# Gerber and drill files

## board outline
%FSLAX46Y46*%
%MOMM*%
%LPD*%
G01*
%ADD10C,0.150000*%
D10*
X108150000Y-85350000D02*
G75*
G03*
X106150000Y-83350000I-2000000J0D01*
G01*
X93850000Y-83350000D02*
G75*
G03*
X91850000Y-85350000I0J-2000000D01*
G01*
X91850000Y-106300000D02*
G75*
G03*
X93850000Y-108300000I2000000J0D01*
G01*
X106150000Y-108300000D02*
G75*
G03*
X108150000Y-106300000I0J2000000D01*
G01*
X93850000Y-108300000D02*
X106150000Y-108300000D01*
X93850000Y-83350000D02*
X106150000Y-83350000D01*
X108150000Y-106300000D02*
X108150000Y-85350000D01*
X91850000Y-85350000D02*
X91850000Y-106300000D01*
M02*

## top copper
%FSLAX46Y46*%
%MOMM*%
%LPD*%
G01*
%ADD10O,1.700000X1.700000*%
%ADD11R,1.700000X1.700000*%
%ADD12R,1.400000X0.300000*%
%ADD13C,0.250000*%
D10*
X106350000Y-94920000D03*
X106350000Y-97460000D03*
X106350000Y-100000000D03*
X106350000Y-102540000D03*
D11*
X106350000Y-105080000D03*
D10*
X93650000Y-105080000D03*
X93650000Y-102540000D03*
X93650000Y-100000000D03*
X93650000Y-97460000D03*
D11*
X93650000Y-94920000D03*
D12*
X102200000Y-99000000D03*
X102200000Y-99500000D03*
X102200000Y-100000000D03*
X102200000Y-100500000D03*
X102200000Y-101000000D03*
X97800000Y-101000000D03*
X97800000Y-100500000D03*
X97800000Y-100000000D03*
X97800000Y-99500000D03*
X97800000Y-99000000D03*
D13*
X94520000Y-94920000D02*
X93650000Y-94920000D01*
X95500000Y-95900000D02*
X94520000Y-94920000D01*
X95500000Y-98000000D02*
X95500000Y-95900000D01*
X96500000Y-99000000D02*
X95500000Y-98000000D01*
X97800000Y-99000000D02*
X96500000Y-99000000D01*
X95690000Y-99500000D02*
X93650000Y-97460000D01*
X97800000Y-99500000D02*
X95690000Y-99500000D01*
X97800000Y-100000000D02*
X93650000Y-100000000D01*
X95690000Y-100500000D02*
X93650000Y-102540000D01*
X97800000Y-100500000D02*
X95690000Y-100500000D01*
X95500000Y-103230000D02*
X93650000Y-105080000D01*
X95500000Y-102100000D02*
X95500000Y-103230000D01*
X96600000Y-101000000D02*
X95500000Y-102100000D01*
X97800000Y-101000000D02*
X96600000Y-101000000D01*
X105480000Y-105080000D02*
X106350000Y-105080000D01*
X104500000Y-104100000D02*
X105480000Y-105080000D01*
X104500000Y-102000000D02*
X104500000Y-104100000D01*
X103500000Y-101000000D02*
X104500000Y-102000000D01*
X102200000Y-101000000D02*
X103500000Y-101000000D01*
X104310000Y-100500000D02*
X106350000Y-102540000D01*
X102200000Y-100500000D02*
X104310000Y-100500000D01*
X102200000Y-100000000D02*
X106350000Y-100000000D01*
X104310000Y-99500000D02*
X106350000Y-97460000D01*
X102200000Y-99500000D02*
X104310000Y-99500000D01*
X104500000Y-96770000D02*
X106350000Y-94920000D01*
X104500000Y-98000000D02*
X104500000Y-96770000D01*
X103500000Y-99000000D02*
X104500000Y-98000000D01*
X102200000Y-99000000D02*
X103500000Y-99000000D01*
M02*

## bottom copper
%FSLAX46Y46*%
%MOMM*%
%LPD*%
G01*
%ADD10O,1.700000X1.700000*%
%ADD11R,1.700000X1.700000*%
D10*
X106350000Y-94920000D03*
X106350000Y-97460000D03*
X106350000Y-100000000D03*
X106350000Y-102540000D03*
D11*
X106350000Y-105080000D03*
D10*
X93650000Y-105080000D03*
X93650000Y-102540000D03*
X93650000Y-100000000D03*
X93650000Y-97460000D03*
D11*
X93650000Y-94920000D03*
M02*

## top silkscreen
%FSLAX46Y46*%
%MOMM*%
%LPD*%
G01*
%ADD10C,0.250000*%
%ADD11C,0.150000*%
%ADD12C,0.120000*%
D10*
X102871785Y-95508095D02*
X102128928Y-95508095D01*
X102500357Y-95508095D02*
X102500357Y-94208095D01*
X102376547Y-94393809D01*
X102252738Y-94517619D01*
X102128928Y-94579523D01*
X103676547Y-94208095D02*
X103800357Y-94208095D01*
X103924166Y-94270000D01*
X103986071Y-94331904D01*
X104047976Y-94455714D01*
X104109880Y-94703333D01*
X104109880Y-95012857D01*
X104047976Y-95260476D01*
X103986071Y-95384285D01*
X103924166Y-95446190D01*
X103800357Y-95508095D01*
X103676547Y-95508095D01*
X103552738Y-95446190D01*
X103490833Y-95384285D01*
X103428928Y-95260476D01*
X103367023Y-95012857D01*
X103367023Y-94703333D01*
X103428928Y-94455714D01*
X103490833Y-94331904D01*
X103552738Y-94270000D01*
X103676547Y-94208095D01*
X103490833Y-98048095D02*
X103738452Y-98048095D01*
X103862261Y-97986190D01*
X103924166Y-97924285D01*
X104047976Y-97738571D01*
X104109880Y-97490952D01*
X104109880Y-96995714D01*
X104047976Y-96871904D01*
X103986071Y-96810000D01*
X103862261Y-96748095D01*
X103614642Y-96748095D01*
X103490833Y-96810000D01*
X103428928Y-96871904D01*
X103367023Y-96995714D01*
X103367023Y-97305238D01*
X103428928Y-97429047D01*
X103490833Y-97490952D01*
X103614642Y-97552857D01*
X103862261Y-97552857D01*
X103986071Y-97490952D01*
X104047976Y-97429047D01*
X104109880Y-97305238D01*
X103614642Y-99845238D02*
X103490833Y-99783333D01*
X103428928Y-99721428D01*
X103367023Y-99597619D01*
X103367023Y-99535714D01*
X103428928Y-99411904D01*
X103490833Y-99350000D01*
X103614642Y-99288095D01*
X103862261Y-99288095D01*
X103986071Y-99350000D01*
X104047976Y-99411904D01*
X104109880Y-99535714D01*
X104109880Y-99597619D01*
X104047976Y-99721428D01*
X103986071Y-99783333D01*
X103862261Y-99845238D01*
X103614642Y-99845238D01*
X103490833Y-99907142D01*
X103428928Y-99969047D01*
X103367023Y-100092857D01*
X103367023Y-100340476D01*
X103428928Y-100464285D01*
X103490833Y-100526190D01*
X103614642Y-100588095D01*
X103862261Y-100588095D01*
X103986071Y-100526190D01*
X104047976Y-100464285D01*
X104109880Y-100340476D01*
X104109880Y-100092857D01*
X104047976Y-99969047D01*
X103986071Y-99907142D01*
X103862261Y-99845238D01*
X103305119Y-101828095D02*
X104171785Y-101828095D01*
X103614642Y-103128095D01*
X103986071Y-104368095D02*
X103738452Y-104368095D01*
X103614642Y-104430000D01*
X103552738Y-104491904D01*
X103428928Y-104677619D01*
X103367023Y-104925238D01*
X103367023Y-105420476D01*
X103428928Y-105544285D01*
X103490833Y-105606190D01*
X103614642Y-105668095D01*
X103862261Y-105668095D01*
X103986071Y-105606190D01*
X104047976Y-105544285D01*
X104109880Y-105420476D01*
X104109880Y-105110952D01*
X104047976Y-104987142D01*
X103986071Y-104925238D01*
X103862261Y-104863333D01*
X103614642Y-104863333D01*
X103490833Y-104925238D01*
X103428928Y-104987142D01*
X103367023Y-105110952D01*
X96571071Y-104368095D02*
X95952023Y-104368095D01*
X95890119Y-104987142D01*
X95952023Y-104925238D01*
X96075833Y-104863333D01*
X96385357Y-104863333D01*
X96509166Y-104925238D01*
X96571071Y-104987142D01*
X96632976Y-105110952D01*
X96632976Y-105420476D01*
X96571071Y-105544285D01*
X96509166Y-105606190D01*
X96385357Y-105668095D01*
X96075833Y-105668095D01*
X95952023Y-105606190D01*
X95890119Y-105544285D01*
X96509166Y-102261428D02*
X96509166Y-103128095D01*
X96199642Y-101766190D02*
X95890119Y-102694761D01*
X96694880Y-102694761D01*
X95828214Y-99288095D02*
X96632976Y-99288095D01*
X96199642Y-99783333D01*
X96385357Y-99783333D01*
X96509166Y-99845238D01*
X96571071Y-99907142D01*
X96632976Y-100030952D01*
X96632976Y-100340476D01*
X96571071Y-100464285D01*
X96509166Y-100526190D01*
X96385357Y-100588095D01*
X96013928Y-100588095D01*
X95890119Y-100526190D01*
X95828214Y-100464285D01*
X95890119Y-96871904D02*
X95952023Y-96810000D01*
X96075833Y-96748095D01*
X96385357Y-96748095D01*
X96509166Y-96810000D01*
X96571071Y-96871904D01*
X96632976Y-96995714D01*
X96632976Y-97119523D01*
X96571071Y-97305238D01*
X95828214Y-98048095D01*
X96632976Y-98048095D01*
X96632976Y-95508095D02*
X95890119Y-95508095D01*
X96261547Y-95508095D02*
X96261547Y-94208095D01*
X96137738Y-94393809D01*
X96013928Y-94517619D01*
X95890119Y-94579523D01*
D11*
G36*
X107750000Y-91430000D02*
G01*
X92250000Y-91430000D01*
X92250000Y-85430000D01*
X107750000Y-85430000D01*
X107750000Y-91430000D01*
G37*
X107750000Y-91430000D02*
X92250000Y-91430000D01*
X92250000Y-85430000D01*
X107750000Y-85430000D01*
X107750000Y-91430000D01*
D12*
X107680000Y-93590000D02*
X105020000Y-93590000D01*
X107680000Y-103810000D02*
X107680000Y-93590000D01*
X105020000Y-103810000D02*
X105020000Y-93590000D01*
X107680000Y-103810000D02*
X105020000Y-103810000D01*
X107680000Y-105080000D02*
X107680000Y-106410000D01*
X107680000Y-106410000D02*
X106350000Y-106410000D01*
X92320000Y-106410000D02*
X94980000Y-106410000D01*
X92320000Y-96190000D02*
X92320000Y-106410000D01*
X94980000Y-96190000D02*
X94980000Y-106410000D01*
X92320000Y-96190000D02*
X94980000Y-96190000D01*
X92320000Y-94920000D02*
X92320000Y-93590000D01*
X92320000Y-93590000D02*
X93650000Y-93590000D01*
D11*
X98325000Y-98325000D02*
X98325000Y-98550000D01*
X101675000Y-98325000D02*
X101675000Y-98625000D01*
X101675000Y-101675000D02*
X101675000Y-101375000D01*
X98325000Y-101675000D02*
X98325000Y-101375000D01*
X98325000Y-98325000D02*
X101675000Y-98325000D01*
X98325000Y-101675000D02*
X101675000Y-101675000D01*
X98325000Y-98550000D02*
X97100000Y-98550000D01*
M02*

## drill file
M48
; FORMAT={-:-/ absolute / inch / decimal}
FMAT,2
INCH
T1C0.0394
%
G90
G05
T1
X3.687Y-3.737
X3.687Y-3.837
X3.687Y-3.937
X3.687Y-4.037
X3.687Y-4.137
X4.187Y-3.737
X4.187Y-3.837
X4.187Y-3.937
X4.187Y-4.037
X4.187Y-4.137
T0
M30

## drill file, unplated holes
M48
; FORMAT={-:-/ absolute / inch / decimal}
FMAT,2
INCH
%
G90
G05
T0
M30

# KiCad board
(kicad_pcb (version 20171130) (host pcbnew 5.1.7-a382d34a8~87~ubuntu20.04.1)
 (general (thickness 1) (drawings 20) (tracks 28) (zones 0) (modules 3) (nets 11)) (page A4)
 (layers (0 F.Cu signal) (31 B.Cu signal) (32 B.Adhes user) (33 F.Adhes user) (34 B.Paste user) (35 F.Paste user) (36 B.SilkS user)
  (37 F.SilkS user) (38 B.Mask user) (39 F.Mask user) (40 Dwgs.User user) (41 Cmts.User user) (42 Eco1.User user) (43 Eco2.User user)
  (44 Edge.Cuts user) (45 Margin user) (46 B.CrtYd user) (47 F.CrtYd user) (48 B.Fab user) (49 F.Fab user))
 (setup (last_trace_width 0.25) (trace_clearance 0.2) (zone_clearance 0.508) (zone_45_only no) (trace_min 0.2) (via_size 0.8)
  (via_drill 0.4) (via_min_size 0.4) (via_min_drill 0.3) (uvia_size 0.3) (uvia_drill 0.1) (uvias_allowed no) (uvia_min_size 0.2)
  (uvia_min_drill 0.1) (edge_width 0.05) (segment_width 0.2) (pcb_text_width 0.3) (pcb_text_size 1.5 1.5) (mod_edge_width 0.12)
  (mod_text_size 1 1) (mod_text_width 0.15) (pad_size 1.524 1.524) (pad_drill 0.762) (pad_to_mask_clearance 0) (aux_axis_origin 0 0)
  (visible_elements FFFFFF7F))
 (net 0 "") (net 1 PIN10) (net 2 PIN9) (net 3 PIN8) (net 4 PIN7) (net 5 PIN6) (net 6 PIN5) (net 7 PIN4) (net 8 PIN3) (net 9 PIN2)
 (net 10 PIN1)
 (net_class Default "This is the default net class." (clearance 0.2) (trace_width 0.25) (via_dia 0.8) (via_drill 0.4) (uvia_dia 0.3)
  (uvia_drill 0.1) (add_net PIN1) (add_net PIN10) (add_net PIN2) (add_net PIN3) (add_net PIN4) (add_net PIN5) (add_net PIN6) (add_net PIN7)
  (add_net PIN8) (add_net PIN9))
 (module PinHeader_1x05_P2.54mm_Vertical (layer F.Cu) (at 106.35 105.08 180)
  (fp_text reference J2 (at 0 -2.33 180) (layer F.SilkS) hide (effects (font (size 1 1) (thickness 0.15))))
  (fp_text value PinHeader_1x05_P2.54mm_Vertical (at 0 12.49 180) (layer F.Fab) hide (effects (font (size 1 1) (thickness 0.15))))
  (fp_line (start -1.33 -1.33) (end 0 -1.33) (layer F.SilkS) (width 0.12))
  (fp_line (start -1.33 0) (end -1.33 -1.33) (layer F.SilkS) (width 0.12))
  (fp_line (start -1.33 1.27) (end 1.33 1.27) (layer F.SilkS) (width 0.12))
  (fp_line (start 1.33 1.27) (end 1.33 11.49) (layer F.SilkS) (width 0.12))
  (fp_line (start -1.33 1.27) (end -1.33 11.49) (layer F.SilkS) (width 0.12))
  (fp_line (start -1.33 11.49) (end 1.33 11.49) (layer F.SilkS) (width 0.12))
  (pad 5 thru_hole oval (at 0 10.16 180) (size 1.7 1.7) (drill 1) (layers *.Cu *.Mask) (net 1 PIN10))
  (pad 4 thru_hole oval (at 0 7.62 180) (size 1.7 1.7) (drill 1) (layers *.Cu *.Mask) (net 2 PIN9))
  (pad 3 thru_hole oval (at 0 5.08 180) (size 1.7 1.7) (drill 1) (layers *.Cu *.Mask) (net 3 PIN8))
  (pad 2 thru_hole oval (at 0 2.54 180) (size 1.7 1.7) (drill 1) (layers *.Cu *.Mask) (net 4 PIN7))
  (pad 1 thru_hole rect (at 0 0 180) (size 1.7 1.7) (drill 1) (layers *.Cu *.Mask) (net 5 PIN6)))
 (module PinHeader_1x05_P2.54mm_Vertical (layer F.Cu) (at 93.65 94.92)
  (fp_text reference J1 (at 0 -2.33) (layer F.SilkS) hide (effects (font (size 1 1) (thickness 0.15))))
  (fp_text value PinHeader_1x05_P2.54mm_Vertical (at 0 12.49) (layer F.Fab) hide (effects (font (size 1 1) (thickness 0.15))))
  (fp_line (start -1.33 -1.33) (end 0 -1.33) (layer F.SilkS) (width 0.12))
  (fp_line (start -1.33 0) (end -1.33 -1.33) (layer F.SilkS) (width 0.12))
  (fp_line (start -1.33 1.27) (end 1.33 1.27) (layer F.SilkS) (width 0.12))
  (fp_line (start 1.33 1.27) (end 1.33 11.49) (layer F.SilkS) (width 0.12))
  (fp_line (start -1.33 1.27) (end -1.33 11.49) (layer F.SilkS) (width 0.12))
  (fp_line (start -1.33 11.49) (end 1.33 11.49) (layer F.SilkS) (width 0.12))
  (pad 5 thru_hole oval (at 0 10.16) (size 1.7 1.7) (drill 1) (layers *.Cu *.Mask) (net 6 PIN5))
  (pad 4 thru_hole oval (at 0 7.62) (size 1.7 1.7) (drill 1) (layers *.Cu *.Mask) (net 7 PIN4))
  (pad 3 thru_hole oval (at 0 5.08) (size 1.7 1.7) (drill 1) (layers *.Cu *.Mask) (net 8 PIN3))
  (pad 2 thru_hole oval (at 0 2.54) (size 1.7 1.7) (drill 1) (layers *.Cu *.Mask) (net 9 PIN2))
  (pad 1 thru_hole rect (at 0 0) (size 1.7 1.7) (drill 1) (layers *.Cu *.Mask) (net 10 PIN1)))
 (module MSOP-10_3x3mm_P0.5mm (layer F.Cu) (at 100 100)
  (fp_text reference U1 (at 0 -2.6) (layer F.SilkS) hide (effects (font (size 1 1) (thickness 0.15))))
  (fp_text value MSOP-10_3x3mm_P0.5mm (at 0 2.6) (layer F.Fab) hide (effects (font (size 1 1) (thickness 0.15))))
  (fp_line (start -1.675 -1.45) (end -2.9 -1.45) (layer F.SilkS) (width 0.15))
  (fp_line (start -1.675 1.675) (end 1.675 1.675) (layer F.SilkS) (width 0.15))
  (fp_line (start -1.675 -1.675) (end 1.675 -1.675) (layer F.SilkS) (width 0.15))
  (fp_line (start -1.675 1.675) (end -1.675 1.375) (layer F.SilkS) (width 0.15))
  (fp_line (start 1.675 1.675) (end 1.675 1.375) (layer F.SilkS) (width 0.15))
  (fp_line (start 1.675 -1.675) (end 1.675 -1.375) (layer F.SilkS) (width 0.15))
  (fp_line (start -1.675 -1.675) (end -1.675 -1.45) (layer F.SilkS) (width 0.15))
  (pad 10 smd rect (at 2.2 -1) (size 1.4 0.3) (layers F.Cu F.Paste F.Mask) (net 1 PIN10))
  (pad 9 smd rect (at 2.2 -0.5) (size 1.4 0.3) (layers F.Cu F.Paste F.Mask) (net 2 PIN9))
  (pad 8 smd rect (at 2.2 0) (size 1.4 0.3) (layers F.Cu F.Paste F.Mask) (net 3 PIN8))
  (pad 7 smd rect (at 2.2 0.5) (size 1.4 0.3) (layers F.Cu F.Paste F.Mask) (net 4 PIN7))
  (pad 6 smd rect (at 2.2 1) (size 1.4 0.3) (layers F.Cu F.Paste F.Mask) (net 5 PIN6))
  (pad 5 smd rect (at -2.2 1) (size 1.4 0.3) (layers F.Cu F.Paste F.Mask) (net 6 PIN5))
  (pad 4 smd rect (at -2.2 0.5) (size 1.4 0.3) (layers F.Cu F.Paste F.Mask) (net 7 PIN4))
  (pad 3 smd rect (at -2.2 0) (size 1.4 0.3) (layers F.Cu F.Paste F.Mask) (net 8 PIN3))
  (pad 2 smd rect (at -2.2 -0.5) (size 1.4 0.3) (layers F.Cu F.Paste F.Mask) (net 9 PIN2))
  (pad 1 smd rect (at -2.2 -1) (size 1.4 0.3) (layers F.Cu F.Paste F.Mask) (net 10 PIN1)))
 (gr_arc (start 106.15 85.35) (end 106.15 83.35) (angle 90) (layer Edge.Cuts) (width 0.15))
 (gr_arc (start 93.85 85.35) (end 91.85 85.35) (angle 90) (layer Edge.Cuts) (width 0.15))
 (gr_arc (start 93.85 106.3) (end 93.85 108.3) (angle 90) (layer Edge.Cuts) (width 0.15))
 (gr_arc (start 106.15 106.3) (end 108.15 106.3) (angle 90) (layer Edge.Cuts) (width 0.15))
 (gr_line (start 93.85 108.3) (end 106.15 108.3) (layer Edge.Cuts) (width 0.15))
 (gr_line (start 93.85 83.35) (end 106.15 83.35) (layer Edge.Cuts) (width 0.15))
 (gr_line (start 108.15 106.3) (end 108.15 85.35) (layer Edge.Cuts) (width 0.15))
 (gr_line (start 91.85 85.35) (end 91.85 106.3) (layer Edge.Cuts) (width 0.15))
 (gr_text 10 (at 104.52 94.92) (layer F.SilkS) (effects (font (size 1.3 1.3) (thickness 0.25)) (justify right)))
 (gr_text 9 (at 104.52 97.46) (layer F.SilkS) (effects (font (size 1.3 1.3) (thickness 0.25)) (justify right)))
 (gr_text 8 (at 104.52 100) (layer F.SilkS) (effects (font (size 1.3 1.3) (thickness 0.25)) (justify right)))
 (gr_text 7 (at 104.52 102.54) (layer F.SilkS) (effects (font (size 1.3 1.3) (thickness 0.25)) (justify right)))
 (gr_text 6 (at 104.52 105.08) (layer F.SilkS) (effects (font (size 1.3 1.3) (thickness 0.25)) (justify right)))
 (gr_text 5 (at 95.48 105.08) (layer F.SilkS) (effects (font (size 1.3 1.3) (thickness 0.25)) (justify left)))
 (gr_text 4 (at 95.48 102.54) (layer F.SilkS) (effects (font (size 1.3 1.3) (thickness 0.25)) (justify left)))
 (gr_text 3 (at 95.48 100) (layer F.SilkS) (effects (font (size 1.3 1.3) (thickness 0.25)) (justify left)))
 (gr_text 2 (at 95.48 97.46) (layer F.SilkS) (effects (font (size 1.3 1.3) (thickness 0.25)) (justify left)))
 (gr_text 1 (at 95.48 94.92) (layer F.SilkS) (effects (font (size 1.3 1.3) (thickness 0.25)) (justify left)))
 (gr_poly (pts (xy 92.25 85.43) (xy 92.25 91.43) (xy 107.75 91.43) (xy 107.75 85.43)) (layer F.SilkS) (width 0.15))
 (segment (start 94.52 94.92) (end 93.65 94.92) (width 0.25) (layer F.Cu) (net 10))
 (segment (start 95.5 95.9) (end 94.52 94.92) (width 0.25) (layer F.Cu) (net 10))
 (segment (start 95.5 98) (end 95.5 95.9) (width 0.25) (layer F.Cu) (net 10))
 (segment (start 96.5 99) (end 95.5 98) (width 0.25) (layer F.Cu) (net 10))
 (segment (start 97.8 99) (end 96.5 99) (width 0.25) (layer F.Cu) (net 10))
 (segment (start 95.69 99.5) (end 93.65 97.46) (width 0.25) (layer F.Cu) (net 9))
 (segment (start 97.8 99.5) (end 95.69 99.5) (width 0.25) (layer F.Cu) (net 9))
 (segment (start 97.8 100) (end 93.65 100) (width 0.25) (layer F.Cu) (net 8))
 (segment (start 95.69 100.5) (end 93.65 102.54) (width 0.25) (layer F.Cu) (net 7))
 (segment (start 97.8 100.5) (end 95.69 100.5) (width 0.25) (layer F.Cu) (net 7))
 (segment (start 95.5 103.23) (end 93.65 105.08) (width 0.25) (layer F.Cu) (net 6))
 (segment (start 95.5 102.1) (end 95.5 103.23) (width 0.25) (layer F.Cu) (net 6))
 (segment (start 96.6 101) (end 95.5 102.1) (width 0.25) (layer F.Cu) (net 6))
 (segment (start 97.8 101) (end 96.6 101) (width 0.25) (layer F.Cu) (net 6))
 (segment (start 105.48 105.08) (end 106.35 105.08) (width 0.25) (layer F.Cu) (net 5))
 (segment (start 104.5 104.1) (end 105.48 105.08) (width 0.25) (layer F.Cu) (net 5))
 (segment (start 104.5 102) (end 104.5 104.1) (width 0.25) (layer F.Cu) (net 5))
 (segment (start 103.5 101) (end 104.5 102) (width 0.25) (layer F.Cu) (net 5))
 (segment (start 102.2 101) (end 103.5 101) (width 0.25) (layer F.Cu) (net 5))
 (segment (start 104.31 100.5) (end 106.35 102.54) (width 0.25) (layer F.Cu) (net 4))
 (segment (start 102.2 100.5) (end 104.31 100.5) (width 0.25) (layer F.Cu) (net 4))
 (segment (start 102.2 100) (end 106.35 100) (width 0.25) (layer F.Cu) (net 3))
 (segment (start 104.31 99.5) (end 106.35 97.46) (width 0.25) (layer F.Cu) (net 2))
 (segment (start 102.2 99.5) (end 104.31 99.5) (width 0.25) (layer F.Cu) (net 2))
 (segment (start 104.5 96.77) (end 106.35 94.92) (width 0.25) (layer F.Cu) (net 1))
 (segment (start 104.5 98) (end 104.5 96.77) (width 0.25) (layer F.Cu) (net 1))
 (segment (start 103.5 99) (end 104.5 98) (width 0.25) (layer F.Cu) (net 1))
 (segment (start 102.2 99) (end 103.5 99) (width 0.25) (layer F.Cu) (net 1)))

